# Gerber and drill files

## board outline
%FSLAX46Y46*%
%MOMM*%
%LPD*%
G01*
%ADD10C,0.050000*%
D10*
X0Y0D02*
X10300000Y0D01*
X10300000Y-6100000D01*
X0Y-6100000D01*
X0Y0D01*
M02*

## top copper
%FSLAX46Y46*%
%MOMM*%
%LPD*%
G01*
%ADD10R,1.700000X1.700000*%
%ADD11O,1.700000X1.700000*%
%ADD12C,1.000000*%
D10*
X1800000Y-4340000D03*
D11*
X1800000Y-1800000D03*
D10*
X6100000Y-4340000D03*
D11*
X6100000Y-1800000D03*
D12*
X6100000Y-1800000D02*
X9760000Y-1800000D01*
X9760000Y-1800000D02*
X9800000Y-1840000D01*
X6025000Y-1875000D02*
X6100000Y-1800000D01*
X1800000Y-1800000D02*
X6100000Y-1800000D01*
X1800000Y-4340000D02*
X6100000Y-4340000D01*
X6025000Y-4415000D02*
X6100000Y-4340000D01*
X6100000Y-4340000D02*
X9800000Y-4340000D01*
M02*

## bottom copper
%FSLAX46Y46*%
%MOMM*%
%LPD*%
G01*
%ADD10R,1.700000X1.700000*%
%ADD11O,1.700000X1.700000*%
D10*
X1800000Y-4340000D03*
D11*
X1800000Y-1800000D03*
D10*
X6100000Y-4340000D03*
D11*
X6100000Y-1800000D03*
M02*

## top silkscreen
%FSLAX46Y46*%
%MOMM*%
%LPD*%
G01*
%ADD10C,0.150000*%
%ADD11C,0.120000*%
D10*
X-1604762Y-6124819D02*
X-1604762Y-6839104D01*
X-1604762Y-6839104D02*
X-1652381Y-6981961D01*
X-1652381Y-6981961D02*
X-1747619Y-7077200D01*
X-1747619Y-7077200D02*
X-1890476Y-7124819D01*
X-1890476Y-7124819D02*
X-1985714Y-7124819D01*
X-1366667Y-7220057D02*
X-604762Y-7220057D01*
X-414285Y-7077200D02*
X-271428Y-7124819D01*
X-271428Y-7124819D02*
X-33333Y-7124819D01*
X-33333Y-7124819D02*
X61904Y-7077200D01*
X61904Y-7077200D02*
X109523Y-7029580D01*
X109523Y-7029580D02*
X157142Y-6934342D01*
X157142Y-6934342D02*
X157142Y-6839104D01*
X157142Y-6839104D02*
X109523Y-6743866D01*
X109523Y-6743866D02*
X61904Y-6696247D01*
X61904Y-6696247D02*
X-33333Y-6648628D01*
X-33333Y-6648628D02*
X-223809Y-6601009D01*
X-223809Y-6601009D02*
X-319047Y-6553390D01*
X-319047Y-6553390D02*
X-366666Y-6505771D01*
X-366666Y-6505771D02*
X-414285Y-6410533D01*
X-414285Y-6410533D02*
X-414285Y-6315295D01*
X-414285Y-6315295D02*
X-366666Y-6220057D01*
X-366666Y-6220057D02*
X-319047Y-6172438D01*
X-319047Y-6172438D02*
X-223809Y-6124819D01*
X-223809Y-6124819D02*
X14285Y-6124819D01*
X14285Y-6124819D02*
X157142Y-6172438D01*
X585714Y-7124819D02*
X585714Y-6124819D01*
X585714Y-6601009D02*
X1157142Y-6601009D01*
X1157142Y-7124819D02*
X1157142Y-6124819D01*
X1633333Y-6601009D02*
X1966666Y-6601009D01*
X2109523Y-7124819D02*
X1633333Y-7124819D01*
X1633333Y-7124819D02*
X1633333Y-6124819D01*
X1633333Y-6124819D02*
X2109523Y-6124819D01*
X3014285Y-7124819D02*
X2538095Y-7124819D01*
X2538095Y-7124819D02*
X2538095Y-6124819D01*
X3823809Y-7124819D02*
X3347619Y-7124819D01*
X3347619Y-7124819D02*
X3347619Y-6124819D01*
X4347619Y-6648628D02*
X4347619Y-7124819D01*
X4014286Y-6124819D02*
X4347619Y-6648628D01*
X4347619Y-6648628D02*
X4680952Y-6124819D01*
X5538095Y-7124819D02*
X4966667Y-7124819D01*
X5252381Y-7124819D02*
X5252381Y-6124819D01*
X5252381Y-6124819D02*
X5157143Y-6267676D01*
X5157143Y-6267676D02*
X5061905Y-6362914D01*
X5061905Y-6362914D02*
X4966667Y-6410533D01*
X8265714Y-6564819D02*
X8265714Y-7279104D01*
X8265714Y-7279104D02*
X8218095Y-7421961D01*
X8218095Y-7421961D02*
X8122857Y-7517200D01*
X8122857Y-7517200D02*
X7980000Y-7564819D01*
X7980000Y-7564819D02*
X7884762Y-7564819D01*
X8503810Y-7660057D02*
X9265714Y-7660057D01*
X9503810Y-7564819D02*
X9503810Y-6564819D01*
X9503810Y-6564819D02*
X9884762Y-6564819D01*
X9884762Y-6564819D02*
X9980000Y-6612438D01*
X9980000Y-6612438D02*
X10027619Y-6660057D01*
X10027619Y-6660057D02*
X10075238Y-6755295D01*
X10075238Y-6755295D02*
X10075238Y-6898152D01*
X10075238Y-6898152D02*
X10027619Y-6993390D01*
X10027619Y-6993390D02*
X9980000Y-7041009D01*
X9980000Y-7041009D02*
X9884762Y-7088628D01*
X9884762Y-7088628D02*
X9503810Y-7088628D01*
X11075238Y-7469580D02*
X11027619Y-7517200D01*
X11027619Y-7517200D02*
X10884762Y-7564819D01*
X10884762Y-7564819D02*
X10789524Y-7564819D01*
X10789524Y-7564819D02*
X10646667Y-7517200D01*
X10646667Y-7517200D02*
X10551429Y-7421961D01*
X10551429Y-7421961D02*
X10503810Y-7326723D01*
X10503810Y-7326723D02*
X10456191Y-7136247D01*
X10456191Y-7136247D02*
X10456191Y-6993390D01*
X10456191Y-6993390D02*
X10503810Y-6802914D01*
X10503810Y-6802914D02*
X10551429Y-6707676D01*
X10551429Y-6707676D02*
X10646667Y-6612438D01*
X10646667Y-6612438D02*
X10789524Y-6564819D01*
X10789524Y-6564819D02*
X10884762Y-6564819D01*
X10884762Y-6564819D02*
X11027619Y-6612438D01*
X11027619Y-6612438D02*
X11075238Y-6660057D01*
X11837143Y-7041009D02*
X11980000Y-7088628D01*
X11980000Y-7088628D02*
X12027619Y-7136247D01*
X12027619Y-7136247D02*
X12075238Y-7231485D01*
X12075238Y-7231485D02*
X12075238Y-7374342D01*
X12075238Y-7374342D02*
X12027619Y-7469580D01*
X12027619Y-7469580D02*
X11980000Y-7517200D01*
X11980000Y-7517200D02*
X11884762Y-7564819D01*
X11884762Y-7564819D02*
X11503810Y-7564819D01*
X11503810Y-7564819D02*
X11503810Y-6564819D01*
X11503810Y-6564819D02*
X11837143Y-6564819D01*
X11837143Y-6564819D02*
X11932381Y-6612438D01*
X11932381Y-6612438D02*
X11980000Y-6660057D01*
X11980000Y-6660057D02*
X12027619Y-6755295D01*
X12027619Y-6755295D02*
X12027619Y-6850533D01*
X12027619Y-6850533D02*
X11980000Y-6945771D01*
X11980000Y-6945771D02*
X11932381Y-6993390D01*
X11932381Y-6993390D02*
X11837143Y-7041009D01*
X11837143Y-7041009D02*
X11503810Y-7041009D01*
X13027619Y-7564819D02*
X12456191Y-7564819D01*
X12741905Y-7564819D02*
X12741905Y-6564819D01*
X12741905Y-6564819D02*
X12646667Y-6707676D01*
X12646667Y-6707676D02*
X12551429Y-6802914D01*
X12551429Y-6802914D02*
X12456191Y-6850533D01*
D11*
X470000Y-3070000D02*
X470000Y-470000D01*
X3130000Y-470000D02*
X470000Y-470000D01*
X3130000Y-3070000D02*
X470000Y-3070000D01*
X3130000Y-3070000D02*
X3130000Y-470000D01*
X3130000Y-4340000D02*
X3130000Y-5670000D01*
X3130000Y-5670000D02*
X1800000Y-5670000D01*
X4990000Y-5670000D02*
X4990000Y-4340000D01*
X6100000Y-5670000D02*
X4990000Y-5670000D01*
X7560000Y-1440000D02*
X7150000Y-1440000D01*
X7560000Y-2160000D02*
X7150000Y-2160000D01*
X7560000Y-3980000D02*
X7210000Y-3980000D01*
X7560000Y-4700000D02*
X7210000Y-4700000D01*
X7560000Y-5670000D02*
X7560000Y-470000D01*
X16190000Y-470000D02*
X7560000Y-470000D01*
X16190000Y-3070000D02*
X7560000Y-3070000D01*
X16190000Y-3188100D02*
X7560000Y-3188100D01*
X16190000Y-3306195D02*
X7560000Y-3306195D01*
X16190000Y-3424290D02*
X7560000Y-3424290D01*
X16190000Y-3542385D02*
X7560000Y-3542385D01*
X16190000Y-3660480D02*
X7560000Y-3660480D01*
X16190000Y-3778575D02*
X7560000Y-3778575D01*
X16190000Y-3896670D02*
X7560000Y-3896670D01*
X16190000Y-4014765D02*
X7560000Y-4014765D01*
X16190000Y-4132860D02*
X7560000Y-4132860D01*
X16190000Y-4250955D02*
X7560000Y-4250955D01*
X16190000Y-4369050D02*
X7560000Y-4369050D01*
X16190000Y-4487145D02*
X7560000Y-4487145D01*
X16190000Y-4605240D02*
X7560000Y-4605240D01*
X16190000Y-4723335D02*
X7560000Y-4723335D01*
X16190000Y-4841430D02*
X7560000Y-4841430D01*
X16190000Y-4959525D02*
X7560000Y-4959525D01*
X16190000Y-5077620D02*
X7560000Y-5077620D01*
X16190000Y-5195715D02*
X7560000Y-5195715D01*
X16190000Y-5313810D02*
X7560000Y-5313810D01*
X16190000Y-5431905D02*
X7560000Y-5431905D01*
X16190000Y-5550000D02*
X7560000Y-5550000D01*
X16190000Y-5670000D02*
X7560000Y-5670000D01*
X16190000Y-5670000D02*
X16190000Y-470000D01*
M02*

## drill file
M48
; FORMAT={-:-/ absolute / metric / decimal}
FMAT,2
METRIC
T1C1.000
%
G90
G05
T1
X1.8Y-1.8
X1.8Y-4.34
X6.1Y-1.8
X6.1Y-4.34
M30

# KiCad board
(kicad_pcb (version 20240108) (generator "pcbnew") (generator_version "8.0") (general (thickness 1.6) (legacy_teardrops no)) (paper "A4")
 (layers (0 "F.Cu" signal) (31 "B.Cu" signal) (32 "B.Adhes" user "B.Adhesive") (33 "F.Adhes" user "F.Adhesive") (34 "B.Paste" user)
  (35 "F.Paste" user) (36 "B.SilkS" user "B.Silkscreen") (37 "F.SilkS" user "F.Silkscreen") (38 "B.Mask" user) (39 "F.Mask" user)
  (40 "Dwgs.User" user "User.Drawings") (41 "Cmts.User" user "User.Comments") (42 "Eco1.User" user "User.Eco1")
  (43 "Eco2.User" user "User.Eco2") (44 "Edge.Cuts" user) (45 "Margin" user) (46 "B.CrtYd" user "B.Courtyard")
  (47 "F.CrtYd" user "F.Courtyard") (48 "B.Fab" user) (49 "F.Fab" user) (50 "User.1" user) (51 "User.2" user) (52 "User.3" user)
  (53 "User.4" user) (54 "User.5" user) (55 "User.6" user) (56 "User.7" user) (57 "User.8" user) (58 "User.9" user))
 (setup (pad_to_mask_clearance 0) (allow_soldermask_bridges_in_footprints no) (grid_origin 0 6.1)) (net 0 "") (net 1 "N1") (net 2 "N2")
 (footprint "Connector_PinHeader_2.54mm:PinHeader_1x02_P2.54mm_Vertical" (layer "F.Cu") (at 1.8 4.34 180)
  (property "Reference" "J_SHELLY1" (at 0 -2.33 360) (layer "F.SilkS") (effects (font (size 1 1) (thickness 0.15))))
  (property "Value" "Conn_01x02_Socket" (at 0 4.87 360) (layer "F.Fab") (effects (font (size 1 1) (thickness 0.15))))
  (fp_line (start 1.33 1.27) (end 1.33 3.87) (stroke (width 0.12) (type solid)) (layer "F.SilkS"))
  (fp_line (start -1.33 3.87) (end 1.33 3.87) (stroke (width 0.12) (type solid)) (layer "F.SilkS"))
  (fp_line (start -1.33 1.27) (end 1.33 1.27) (stroke (width 0.12) (type solid)) (layer "F.SilkS"))
  (fp_line (start -1.33 1.27) (end -1.33 3.87) (stroke (width 0.12) (type solid)) (layer "F.SilkS"))
  (fp_line (start -1.33 0) (end -1.33 -1.33) (stroke (width 0.12) (type solid)) (layer "F.SilkS"))
  (fp_line (start -1.33 -1.33) (end 0 -1.33) (stroke (width 0.12) (type solid)) (layer "F.SilkS"))
  (pad "1" thru_hole rect (at 0 0 180) (size 1.7 1.7) (drill 1) (layers "*.Cu" "*.Mask") (remove_unused_layers no) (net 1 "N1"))
  (pad "2" thru_hole oval (at 0 2.54 180) (size 1.7 1.7) (drill 1) (layers "*.Cu" "*.Mask") (remove_unused_layers no) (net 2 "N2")))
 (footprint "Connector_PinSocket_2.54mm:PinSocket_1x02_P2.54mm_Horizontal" (layer "F.Cu") (at 6.1 4.34 180)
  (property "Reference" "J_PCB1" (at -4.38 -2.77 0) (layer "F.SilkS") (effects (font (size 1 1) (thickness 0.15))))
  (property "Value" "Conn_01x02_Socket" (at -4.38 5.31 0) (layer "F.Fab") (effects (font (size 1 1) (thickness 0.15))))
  (fp_line (start 1.11 -1.33) (end 1.11 0) (stroke (width 0.12) (type solid)) (layer "F.SilkS"))
  (fp_line (start 0 -1.33) (end 1.11 -1.33) (stroke (width 0.12) (type solid)) (layer "F.SilkS"))
  (fp_line (start -1.46 2.9) (end -1.05 2.9) (stroke (width 0.12) (type solid)) (layer "F.SilkS"))
  (fp_line (start -1.46 2.18) (end -1.05 2.18) (stroke (width 0.12) (type solid)) (layer "F.SilkS"))
  (fp_line (start -1.46 0.36) (end -1.11 0.36) (stroke (width 0.12) (type solid)) (layer "F.SilkS"))
  (fp_line (start -1.46 -0.36) (end -1.11 -0.36) (stroke (width 0.12) (type solid)) (layer "F.SilkS"))
  (fp_line (start -1.46 -1.33) (end -1.46 3.87) (stroke (width 0.12) (type solid)) (layer "F.SilkS"))
  (fp_line (start -10.09 3.87) (end -1.46 3.87) (stroke (width 0.12) (type solid)) (layer "F.SilkS"))
  (fp_line (start -10.09 1.27) (end -1.46 1.27) (stroke (width 0.12) (type solid)) (layer "F.SilkS"))
  (fp_line (start -10.09 1.1519) (end -1.46 1.1519) (stroke (width 0.12) (type solid)) (layer "F.SilkS"))
  (fp_line (start -10.09 1.033805) (end -1.46 1.033805) (stroke (width 0.12) (type solid)) (layer "F.SilkS"))
  (fp_line (start -10.09 0.91571) (end -1.46 0.91571) (stroke (width 0.12) (type solid)) (layer "F.SilkS"))
  (fp_line (start -10.09 0.797615) (end -1.46 0.797615) (stroke (width 0.12) (type solid)) (layer "F.SilkS"))
  (fp_line (start -10.09 0.67952) (end -1.46 0.67952) (stroke (width 0.12) (type solid)) (layer "F.SilkS"))
  (fp_line (start -10.09 0.561425) (end -1.46 0.561425) (stroke (width 0.12) (type solid)) (layer "F.SilkS"))
  (fp_line (start -10.09 0.44333) (end -1.46 0.44333) (stroke (width 0.12) (type solid)) (layer "F.SilkS"))
  (fp_line (start -10.09 0.325235) (end -1.46 0.325235) (stroke (width 0.12) (type solid)) (layer "F.SilkS"))
  (fp_line (start -10.09 0.20714) (end -1.46 0.20714) (stroke (width 0.12) (type solid)) (layer "F.SilkS"))
  (fp_line (start -10.09 0.089045) (end -1.46 0.089045) (stroke (width 0.12) (type solid)) (layer "F.SilkS"))
  (fp_line (start -10.09 -0.02905) (end -1.46 -0.02905) (stroke (width 0.12) (type solid)) (layer "F.SilkS"))
  (fp_line (start -10.09 -0.147145) (end -1.46 -0.147145) (stroke (width 0.12) (type solid)) (layer "F.SilkS"))
  (fp_line (start -10.09 -0.26524) (end -1.46 -0.26524) (stroke (width 0.12) (type solid)) (layer "F.SilkS"))
  (fp_line (start -10.09 -0.383335) (end -1.46 -0.383335) (stroke (width 0.12) (type solid)) (layer "F.SilkS"))
  (fp_line (start -10.09 -0.50143) (end -1.46 -0.50143) (stroke (width 0.12) (type solid)) (layer "F.SilkS"))
  (fp_line (start -10.09 -0.619525) (end -1.46 -0.619525) (stroke (width 0.12) (type solid)) (layer "F.SilkS"))
  (fp_line (start -10.09 -0.73762) (end -1.46 -0.73762) (stroke (width 0.12) (type solid)) (layer "F.SilkS"))
  (fp_line (start -10.09 -0.855715) (end -1.46 -0.855715) (stroke (width 0.12) (type solid)) (layer "F.SilkS"))
  (fp_line (start -10.09 -0.97381) (end -1.46 -0.97381) (stroke (width 0.12) (type solid)) (layer "F.SilkS"))
  (fp_line (start -10.09 -1.091905) (end -1.46 -1.091905) (stroke (width 0.12) (type solid)) (layer "F.SilkS"))
  (fp_line (start -10.09 -1.21) (end -1.46 -1.21) (stroke (width 0.12) (type solid)) (layer "F.SilkS"))
  (fp_line (start -10.09 -1.33) (end -1.46 -1.33) (stroke (width 0.12) (type solid)) (layer "F.SilkS"))
  (fp_line (start -10.09 -1.33) (end -10.09 3.87) (stroke (width 0.12) (type solid)) (layer "F.SilkS"))
  (pad "1" thru_hole rect (at 0 0 180) (size 1.7 1.7) (drill 1) (layers "*.Cu" "*.Mask") (remove_unused_layers no) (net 1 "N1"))
  (pad "2" thru_hole oval (at 0 2.54 180) (size 1.7 1.7) (drill 1) (layers "*.Cu" "*.Mask") (remove_unused_layers no) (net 2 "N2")))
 (gr_rect (start 0 0) (end 10.3 6.1) (stroke (width 0.05) (type default)) (fill none) (layer "Edge.Cuts"))
 (segment (start 6.1 1.8) (end 9.76 1.8) (width 1) (layer "F.Cu") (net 2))
 (segment (start 9.76 1.8) (end 9.8 1.84) (width 1) (layer "F.Cu") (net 2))
 (segment (start 6.025 1.875) (end 6.1 1.8) (width 1) (layer "F.Cu") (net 2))
 (segment (start 1.8 1.8) (end 6.1 1.8) (width 1) (layer "F.Cu") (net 2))
 (segment (start 1.8 4.34) (end 6.1 4.34) (width 1) (layer "F.Cu") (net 1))
 (segment (start 6.025 4.415) (end 6.1 4.34) (width 1) (layer "F.Cu") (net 1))
 (segment (start 6.1 4.34) (end 9.8 4.34) (width 1) (layer "F.Cu") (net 1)))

